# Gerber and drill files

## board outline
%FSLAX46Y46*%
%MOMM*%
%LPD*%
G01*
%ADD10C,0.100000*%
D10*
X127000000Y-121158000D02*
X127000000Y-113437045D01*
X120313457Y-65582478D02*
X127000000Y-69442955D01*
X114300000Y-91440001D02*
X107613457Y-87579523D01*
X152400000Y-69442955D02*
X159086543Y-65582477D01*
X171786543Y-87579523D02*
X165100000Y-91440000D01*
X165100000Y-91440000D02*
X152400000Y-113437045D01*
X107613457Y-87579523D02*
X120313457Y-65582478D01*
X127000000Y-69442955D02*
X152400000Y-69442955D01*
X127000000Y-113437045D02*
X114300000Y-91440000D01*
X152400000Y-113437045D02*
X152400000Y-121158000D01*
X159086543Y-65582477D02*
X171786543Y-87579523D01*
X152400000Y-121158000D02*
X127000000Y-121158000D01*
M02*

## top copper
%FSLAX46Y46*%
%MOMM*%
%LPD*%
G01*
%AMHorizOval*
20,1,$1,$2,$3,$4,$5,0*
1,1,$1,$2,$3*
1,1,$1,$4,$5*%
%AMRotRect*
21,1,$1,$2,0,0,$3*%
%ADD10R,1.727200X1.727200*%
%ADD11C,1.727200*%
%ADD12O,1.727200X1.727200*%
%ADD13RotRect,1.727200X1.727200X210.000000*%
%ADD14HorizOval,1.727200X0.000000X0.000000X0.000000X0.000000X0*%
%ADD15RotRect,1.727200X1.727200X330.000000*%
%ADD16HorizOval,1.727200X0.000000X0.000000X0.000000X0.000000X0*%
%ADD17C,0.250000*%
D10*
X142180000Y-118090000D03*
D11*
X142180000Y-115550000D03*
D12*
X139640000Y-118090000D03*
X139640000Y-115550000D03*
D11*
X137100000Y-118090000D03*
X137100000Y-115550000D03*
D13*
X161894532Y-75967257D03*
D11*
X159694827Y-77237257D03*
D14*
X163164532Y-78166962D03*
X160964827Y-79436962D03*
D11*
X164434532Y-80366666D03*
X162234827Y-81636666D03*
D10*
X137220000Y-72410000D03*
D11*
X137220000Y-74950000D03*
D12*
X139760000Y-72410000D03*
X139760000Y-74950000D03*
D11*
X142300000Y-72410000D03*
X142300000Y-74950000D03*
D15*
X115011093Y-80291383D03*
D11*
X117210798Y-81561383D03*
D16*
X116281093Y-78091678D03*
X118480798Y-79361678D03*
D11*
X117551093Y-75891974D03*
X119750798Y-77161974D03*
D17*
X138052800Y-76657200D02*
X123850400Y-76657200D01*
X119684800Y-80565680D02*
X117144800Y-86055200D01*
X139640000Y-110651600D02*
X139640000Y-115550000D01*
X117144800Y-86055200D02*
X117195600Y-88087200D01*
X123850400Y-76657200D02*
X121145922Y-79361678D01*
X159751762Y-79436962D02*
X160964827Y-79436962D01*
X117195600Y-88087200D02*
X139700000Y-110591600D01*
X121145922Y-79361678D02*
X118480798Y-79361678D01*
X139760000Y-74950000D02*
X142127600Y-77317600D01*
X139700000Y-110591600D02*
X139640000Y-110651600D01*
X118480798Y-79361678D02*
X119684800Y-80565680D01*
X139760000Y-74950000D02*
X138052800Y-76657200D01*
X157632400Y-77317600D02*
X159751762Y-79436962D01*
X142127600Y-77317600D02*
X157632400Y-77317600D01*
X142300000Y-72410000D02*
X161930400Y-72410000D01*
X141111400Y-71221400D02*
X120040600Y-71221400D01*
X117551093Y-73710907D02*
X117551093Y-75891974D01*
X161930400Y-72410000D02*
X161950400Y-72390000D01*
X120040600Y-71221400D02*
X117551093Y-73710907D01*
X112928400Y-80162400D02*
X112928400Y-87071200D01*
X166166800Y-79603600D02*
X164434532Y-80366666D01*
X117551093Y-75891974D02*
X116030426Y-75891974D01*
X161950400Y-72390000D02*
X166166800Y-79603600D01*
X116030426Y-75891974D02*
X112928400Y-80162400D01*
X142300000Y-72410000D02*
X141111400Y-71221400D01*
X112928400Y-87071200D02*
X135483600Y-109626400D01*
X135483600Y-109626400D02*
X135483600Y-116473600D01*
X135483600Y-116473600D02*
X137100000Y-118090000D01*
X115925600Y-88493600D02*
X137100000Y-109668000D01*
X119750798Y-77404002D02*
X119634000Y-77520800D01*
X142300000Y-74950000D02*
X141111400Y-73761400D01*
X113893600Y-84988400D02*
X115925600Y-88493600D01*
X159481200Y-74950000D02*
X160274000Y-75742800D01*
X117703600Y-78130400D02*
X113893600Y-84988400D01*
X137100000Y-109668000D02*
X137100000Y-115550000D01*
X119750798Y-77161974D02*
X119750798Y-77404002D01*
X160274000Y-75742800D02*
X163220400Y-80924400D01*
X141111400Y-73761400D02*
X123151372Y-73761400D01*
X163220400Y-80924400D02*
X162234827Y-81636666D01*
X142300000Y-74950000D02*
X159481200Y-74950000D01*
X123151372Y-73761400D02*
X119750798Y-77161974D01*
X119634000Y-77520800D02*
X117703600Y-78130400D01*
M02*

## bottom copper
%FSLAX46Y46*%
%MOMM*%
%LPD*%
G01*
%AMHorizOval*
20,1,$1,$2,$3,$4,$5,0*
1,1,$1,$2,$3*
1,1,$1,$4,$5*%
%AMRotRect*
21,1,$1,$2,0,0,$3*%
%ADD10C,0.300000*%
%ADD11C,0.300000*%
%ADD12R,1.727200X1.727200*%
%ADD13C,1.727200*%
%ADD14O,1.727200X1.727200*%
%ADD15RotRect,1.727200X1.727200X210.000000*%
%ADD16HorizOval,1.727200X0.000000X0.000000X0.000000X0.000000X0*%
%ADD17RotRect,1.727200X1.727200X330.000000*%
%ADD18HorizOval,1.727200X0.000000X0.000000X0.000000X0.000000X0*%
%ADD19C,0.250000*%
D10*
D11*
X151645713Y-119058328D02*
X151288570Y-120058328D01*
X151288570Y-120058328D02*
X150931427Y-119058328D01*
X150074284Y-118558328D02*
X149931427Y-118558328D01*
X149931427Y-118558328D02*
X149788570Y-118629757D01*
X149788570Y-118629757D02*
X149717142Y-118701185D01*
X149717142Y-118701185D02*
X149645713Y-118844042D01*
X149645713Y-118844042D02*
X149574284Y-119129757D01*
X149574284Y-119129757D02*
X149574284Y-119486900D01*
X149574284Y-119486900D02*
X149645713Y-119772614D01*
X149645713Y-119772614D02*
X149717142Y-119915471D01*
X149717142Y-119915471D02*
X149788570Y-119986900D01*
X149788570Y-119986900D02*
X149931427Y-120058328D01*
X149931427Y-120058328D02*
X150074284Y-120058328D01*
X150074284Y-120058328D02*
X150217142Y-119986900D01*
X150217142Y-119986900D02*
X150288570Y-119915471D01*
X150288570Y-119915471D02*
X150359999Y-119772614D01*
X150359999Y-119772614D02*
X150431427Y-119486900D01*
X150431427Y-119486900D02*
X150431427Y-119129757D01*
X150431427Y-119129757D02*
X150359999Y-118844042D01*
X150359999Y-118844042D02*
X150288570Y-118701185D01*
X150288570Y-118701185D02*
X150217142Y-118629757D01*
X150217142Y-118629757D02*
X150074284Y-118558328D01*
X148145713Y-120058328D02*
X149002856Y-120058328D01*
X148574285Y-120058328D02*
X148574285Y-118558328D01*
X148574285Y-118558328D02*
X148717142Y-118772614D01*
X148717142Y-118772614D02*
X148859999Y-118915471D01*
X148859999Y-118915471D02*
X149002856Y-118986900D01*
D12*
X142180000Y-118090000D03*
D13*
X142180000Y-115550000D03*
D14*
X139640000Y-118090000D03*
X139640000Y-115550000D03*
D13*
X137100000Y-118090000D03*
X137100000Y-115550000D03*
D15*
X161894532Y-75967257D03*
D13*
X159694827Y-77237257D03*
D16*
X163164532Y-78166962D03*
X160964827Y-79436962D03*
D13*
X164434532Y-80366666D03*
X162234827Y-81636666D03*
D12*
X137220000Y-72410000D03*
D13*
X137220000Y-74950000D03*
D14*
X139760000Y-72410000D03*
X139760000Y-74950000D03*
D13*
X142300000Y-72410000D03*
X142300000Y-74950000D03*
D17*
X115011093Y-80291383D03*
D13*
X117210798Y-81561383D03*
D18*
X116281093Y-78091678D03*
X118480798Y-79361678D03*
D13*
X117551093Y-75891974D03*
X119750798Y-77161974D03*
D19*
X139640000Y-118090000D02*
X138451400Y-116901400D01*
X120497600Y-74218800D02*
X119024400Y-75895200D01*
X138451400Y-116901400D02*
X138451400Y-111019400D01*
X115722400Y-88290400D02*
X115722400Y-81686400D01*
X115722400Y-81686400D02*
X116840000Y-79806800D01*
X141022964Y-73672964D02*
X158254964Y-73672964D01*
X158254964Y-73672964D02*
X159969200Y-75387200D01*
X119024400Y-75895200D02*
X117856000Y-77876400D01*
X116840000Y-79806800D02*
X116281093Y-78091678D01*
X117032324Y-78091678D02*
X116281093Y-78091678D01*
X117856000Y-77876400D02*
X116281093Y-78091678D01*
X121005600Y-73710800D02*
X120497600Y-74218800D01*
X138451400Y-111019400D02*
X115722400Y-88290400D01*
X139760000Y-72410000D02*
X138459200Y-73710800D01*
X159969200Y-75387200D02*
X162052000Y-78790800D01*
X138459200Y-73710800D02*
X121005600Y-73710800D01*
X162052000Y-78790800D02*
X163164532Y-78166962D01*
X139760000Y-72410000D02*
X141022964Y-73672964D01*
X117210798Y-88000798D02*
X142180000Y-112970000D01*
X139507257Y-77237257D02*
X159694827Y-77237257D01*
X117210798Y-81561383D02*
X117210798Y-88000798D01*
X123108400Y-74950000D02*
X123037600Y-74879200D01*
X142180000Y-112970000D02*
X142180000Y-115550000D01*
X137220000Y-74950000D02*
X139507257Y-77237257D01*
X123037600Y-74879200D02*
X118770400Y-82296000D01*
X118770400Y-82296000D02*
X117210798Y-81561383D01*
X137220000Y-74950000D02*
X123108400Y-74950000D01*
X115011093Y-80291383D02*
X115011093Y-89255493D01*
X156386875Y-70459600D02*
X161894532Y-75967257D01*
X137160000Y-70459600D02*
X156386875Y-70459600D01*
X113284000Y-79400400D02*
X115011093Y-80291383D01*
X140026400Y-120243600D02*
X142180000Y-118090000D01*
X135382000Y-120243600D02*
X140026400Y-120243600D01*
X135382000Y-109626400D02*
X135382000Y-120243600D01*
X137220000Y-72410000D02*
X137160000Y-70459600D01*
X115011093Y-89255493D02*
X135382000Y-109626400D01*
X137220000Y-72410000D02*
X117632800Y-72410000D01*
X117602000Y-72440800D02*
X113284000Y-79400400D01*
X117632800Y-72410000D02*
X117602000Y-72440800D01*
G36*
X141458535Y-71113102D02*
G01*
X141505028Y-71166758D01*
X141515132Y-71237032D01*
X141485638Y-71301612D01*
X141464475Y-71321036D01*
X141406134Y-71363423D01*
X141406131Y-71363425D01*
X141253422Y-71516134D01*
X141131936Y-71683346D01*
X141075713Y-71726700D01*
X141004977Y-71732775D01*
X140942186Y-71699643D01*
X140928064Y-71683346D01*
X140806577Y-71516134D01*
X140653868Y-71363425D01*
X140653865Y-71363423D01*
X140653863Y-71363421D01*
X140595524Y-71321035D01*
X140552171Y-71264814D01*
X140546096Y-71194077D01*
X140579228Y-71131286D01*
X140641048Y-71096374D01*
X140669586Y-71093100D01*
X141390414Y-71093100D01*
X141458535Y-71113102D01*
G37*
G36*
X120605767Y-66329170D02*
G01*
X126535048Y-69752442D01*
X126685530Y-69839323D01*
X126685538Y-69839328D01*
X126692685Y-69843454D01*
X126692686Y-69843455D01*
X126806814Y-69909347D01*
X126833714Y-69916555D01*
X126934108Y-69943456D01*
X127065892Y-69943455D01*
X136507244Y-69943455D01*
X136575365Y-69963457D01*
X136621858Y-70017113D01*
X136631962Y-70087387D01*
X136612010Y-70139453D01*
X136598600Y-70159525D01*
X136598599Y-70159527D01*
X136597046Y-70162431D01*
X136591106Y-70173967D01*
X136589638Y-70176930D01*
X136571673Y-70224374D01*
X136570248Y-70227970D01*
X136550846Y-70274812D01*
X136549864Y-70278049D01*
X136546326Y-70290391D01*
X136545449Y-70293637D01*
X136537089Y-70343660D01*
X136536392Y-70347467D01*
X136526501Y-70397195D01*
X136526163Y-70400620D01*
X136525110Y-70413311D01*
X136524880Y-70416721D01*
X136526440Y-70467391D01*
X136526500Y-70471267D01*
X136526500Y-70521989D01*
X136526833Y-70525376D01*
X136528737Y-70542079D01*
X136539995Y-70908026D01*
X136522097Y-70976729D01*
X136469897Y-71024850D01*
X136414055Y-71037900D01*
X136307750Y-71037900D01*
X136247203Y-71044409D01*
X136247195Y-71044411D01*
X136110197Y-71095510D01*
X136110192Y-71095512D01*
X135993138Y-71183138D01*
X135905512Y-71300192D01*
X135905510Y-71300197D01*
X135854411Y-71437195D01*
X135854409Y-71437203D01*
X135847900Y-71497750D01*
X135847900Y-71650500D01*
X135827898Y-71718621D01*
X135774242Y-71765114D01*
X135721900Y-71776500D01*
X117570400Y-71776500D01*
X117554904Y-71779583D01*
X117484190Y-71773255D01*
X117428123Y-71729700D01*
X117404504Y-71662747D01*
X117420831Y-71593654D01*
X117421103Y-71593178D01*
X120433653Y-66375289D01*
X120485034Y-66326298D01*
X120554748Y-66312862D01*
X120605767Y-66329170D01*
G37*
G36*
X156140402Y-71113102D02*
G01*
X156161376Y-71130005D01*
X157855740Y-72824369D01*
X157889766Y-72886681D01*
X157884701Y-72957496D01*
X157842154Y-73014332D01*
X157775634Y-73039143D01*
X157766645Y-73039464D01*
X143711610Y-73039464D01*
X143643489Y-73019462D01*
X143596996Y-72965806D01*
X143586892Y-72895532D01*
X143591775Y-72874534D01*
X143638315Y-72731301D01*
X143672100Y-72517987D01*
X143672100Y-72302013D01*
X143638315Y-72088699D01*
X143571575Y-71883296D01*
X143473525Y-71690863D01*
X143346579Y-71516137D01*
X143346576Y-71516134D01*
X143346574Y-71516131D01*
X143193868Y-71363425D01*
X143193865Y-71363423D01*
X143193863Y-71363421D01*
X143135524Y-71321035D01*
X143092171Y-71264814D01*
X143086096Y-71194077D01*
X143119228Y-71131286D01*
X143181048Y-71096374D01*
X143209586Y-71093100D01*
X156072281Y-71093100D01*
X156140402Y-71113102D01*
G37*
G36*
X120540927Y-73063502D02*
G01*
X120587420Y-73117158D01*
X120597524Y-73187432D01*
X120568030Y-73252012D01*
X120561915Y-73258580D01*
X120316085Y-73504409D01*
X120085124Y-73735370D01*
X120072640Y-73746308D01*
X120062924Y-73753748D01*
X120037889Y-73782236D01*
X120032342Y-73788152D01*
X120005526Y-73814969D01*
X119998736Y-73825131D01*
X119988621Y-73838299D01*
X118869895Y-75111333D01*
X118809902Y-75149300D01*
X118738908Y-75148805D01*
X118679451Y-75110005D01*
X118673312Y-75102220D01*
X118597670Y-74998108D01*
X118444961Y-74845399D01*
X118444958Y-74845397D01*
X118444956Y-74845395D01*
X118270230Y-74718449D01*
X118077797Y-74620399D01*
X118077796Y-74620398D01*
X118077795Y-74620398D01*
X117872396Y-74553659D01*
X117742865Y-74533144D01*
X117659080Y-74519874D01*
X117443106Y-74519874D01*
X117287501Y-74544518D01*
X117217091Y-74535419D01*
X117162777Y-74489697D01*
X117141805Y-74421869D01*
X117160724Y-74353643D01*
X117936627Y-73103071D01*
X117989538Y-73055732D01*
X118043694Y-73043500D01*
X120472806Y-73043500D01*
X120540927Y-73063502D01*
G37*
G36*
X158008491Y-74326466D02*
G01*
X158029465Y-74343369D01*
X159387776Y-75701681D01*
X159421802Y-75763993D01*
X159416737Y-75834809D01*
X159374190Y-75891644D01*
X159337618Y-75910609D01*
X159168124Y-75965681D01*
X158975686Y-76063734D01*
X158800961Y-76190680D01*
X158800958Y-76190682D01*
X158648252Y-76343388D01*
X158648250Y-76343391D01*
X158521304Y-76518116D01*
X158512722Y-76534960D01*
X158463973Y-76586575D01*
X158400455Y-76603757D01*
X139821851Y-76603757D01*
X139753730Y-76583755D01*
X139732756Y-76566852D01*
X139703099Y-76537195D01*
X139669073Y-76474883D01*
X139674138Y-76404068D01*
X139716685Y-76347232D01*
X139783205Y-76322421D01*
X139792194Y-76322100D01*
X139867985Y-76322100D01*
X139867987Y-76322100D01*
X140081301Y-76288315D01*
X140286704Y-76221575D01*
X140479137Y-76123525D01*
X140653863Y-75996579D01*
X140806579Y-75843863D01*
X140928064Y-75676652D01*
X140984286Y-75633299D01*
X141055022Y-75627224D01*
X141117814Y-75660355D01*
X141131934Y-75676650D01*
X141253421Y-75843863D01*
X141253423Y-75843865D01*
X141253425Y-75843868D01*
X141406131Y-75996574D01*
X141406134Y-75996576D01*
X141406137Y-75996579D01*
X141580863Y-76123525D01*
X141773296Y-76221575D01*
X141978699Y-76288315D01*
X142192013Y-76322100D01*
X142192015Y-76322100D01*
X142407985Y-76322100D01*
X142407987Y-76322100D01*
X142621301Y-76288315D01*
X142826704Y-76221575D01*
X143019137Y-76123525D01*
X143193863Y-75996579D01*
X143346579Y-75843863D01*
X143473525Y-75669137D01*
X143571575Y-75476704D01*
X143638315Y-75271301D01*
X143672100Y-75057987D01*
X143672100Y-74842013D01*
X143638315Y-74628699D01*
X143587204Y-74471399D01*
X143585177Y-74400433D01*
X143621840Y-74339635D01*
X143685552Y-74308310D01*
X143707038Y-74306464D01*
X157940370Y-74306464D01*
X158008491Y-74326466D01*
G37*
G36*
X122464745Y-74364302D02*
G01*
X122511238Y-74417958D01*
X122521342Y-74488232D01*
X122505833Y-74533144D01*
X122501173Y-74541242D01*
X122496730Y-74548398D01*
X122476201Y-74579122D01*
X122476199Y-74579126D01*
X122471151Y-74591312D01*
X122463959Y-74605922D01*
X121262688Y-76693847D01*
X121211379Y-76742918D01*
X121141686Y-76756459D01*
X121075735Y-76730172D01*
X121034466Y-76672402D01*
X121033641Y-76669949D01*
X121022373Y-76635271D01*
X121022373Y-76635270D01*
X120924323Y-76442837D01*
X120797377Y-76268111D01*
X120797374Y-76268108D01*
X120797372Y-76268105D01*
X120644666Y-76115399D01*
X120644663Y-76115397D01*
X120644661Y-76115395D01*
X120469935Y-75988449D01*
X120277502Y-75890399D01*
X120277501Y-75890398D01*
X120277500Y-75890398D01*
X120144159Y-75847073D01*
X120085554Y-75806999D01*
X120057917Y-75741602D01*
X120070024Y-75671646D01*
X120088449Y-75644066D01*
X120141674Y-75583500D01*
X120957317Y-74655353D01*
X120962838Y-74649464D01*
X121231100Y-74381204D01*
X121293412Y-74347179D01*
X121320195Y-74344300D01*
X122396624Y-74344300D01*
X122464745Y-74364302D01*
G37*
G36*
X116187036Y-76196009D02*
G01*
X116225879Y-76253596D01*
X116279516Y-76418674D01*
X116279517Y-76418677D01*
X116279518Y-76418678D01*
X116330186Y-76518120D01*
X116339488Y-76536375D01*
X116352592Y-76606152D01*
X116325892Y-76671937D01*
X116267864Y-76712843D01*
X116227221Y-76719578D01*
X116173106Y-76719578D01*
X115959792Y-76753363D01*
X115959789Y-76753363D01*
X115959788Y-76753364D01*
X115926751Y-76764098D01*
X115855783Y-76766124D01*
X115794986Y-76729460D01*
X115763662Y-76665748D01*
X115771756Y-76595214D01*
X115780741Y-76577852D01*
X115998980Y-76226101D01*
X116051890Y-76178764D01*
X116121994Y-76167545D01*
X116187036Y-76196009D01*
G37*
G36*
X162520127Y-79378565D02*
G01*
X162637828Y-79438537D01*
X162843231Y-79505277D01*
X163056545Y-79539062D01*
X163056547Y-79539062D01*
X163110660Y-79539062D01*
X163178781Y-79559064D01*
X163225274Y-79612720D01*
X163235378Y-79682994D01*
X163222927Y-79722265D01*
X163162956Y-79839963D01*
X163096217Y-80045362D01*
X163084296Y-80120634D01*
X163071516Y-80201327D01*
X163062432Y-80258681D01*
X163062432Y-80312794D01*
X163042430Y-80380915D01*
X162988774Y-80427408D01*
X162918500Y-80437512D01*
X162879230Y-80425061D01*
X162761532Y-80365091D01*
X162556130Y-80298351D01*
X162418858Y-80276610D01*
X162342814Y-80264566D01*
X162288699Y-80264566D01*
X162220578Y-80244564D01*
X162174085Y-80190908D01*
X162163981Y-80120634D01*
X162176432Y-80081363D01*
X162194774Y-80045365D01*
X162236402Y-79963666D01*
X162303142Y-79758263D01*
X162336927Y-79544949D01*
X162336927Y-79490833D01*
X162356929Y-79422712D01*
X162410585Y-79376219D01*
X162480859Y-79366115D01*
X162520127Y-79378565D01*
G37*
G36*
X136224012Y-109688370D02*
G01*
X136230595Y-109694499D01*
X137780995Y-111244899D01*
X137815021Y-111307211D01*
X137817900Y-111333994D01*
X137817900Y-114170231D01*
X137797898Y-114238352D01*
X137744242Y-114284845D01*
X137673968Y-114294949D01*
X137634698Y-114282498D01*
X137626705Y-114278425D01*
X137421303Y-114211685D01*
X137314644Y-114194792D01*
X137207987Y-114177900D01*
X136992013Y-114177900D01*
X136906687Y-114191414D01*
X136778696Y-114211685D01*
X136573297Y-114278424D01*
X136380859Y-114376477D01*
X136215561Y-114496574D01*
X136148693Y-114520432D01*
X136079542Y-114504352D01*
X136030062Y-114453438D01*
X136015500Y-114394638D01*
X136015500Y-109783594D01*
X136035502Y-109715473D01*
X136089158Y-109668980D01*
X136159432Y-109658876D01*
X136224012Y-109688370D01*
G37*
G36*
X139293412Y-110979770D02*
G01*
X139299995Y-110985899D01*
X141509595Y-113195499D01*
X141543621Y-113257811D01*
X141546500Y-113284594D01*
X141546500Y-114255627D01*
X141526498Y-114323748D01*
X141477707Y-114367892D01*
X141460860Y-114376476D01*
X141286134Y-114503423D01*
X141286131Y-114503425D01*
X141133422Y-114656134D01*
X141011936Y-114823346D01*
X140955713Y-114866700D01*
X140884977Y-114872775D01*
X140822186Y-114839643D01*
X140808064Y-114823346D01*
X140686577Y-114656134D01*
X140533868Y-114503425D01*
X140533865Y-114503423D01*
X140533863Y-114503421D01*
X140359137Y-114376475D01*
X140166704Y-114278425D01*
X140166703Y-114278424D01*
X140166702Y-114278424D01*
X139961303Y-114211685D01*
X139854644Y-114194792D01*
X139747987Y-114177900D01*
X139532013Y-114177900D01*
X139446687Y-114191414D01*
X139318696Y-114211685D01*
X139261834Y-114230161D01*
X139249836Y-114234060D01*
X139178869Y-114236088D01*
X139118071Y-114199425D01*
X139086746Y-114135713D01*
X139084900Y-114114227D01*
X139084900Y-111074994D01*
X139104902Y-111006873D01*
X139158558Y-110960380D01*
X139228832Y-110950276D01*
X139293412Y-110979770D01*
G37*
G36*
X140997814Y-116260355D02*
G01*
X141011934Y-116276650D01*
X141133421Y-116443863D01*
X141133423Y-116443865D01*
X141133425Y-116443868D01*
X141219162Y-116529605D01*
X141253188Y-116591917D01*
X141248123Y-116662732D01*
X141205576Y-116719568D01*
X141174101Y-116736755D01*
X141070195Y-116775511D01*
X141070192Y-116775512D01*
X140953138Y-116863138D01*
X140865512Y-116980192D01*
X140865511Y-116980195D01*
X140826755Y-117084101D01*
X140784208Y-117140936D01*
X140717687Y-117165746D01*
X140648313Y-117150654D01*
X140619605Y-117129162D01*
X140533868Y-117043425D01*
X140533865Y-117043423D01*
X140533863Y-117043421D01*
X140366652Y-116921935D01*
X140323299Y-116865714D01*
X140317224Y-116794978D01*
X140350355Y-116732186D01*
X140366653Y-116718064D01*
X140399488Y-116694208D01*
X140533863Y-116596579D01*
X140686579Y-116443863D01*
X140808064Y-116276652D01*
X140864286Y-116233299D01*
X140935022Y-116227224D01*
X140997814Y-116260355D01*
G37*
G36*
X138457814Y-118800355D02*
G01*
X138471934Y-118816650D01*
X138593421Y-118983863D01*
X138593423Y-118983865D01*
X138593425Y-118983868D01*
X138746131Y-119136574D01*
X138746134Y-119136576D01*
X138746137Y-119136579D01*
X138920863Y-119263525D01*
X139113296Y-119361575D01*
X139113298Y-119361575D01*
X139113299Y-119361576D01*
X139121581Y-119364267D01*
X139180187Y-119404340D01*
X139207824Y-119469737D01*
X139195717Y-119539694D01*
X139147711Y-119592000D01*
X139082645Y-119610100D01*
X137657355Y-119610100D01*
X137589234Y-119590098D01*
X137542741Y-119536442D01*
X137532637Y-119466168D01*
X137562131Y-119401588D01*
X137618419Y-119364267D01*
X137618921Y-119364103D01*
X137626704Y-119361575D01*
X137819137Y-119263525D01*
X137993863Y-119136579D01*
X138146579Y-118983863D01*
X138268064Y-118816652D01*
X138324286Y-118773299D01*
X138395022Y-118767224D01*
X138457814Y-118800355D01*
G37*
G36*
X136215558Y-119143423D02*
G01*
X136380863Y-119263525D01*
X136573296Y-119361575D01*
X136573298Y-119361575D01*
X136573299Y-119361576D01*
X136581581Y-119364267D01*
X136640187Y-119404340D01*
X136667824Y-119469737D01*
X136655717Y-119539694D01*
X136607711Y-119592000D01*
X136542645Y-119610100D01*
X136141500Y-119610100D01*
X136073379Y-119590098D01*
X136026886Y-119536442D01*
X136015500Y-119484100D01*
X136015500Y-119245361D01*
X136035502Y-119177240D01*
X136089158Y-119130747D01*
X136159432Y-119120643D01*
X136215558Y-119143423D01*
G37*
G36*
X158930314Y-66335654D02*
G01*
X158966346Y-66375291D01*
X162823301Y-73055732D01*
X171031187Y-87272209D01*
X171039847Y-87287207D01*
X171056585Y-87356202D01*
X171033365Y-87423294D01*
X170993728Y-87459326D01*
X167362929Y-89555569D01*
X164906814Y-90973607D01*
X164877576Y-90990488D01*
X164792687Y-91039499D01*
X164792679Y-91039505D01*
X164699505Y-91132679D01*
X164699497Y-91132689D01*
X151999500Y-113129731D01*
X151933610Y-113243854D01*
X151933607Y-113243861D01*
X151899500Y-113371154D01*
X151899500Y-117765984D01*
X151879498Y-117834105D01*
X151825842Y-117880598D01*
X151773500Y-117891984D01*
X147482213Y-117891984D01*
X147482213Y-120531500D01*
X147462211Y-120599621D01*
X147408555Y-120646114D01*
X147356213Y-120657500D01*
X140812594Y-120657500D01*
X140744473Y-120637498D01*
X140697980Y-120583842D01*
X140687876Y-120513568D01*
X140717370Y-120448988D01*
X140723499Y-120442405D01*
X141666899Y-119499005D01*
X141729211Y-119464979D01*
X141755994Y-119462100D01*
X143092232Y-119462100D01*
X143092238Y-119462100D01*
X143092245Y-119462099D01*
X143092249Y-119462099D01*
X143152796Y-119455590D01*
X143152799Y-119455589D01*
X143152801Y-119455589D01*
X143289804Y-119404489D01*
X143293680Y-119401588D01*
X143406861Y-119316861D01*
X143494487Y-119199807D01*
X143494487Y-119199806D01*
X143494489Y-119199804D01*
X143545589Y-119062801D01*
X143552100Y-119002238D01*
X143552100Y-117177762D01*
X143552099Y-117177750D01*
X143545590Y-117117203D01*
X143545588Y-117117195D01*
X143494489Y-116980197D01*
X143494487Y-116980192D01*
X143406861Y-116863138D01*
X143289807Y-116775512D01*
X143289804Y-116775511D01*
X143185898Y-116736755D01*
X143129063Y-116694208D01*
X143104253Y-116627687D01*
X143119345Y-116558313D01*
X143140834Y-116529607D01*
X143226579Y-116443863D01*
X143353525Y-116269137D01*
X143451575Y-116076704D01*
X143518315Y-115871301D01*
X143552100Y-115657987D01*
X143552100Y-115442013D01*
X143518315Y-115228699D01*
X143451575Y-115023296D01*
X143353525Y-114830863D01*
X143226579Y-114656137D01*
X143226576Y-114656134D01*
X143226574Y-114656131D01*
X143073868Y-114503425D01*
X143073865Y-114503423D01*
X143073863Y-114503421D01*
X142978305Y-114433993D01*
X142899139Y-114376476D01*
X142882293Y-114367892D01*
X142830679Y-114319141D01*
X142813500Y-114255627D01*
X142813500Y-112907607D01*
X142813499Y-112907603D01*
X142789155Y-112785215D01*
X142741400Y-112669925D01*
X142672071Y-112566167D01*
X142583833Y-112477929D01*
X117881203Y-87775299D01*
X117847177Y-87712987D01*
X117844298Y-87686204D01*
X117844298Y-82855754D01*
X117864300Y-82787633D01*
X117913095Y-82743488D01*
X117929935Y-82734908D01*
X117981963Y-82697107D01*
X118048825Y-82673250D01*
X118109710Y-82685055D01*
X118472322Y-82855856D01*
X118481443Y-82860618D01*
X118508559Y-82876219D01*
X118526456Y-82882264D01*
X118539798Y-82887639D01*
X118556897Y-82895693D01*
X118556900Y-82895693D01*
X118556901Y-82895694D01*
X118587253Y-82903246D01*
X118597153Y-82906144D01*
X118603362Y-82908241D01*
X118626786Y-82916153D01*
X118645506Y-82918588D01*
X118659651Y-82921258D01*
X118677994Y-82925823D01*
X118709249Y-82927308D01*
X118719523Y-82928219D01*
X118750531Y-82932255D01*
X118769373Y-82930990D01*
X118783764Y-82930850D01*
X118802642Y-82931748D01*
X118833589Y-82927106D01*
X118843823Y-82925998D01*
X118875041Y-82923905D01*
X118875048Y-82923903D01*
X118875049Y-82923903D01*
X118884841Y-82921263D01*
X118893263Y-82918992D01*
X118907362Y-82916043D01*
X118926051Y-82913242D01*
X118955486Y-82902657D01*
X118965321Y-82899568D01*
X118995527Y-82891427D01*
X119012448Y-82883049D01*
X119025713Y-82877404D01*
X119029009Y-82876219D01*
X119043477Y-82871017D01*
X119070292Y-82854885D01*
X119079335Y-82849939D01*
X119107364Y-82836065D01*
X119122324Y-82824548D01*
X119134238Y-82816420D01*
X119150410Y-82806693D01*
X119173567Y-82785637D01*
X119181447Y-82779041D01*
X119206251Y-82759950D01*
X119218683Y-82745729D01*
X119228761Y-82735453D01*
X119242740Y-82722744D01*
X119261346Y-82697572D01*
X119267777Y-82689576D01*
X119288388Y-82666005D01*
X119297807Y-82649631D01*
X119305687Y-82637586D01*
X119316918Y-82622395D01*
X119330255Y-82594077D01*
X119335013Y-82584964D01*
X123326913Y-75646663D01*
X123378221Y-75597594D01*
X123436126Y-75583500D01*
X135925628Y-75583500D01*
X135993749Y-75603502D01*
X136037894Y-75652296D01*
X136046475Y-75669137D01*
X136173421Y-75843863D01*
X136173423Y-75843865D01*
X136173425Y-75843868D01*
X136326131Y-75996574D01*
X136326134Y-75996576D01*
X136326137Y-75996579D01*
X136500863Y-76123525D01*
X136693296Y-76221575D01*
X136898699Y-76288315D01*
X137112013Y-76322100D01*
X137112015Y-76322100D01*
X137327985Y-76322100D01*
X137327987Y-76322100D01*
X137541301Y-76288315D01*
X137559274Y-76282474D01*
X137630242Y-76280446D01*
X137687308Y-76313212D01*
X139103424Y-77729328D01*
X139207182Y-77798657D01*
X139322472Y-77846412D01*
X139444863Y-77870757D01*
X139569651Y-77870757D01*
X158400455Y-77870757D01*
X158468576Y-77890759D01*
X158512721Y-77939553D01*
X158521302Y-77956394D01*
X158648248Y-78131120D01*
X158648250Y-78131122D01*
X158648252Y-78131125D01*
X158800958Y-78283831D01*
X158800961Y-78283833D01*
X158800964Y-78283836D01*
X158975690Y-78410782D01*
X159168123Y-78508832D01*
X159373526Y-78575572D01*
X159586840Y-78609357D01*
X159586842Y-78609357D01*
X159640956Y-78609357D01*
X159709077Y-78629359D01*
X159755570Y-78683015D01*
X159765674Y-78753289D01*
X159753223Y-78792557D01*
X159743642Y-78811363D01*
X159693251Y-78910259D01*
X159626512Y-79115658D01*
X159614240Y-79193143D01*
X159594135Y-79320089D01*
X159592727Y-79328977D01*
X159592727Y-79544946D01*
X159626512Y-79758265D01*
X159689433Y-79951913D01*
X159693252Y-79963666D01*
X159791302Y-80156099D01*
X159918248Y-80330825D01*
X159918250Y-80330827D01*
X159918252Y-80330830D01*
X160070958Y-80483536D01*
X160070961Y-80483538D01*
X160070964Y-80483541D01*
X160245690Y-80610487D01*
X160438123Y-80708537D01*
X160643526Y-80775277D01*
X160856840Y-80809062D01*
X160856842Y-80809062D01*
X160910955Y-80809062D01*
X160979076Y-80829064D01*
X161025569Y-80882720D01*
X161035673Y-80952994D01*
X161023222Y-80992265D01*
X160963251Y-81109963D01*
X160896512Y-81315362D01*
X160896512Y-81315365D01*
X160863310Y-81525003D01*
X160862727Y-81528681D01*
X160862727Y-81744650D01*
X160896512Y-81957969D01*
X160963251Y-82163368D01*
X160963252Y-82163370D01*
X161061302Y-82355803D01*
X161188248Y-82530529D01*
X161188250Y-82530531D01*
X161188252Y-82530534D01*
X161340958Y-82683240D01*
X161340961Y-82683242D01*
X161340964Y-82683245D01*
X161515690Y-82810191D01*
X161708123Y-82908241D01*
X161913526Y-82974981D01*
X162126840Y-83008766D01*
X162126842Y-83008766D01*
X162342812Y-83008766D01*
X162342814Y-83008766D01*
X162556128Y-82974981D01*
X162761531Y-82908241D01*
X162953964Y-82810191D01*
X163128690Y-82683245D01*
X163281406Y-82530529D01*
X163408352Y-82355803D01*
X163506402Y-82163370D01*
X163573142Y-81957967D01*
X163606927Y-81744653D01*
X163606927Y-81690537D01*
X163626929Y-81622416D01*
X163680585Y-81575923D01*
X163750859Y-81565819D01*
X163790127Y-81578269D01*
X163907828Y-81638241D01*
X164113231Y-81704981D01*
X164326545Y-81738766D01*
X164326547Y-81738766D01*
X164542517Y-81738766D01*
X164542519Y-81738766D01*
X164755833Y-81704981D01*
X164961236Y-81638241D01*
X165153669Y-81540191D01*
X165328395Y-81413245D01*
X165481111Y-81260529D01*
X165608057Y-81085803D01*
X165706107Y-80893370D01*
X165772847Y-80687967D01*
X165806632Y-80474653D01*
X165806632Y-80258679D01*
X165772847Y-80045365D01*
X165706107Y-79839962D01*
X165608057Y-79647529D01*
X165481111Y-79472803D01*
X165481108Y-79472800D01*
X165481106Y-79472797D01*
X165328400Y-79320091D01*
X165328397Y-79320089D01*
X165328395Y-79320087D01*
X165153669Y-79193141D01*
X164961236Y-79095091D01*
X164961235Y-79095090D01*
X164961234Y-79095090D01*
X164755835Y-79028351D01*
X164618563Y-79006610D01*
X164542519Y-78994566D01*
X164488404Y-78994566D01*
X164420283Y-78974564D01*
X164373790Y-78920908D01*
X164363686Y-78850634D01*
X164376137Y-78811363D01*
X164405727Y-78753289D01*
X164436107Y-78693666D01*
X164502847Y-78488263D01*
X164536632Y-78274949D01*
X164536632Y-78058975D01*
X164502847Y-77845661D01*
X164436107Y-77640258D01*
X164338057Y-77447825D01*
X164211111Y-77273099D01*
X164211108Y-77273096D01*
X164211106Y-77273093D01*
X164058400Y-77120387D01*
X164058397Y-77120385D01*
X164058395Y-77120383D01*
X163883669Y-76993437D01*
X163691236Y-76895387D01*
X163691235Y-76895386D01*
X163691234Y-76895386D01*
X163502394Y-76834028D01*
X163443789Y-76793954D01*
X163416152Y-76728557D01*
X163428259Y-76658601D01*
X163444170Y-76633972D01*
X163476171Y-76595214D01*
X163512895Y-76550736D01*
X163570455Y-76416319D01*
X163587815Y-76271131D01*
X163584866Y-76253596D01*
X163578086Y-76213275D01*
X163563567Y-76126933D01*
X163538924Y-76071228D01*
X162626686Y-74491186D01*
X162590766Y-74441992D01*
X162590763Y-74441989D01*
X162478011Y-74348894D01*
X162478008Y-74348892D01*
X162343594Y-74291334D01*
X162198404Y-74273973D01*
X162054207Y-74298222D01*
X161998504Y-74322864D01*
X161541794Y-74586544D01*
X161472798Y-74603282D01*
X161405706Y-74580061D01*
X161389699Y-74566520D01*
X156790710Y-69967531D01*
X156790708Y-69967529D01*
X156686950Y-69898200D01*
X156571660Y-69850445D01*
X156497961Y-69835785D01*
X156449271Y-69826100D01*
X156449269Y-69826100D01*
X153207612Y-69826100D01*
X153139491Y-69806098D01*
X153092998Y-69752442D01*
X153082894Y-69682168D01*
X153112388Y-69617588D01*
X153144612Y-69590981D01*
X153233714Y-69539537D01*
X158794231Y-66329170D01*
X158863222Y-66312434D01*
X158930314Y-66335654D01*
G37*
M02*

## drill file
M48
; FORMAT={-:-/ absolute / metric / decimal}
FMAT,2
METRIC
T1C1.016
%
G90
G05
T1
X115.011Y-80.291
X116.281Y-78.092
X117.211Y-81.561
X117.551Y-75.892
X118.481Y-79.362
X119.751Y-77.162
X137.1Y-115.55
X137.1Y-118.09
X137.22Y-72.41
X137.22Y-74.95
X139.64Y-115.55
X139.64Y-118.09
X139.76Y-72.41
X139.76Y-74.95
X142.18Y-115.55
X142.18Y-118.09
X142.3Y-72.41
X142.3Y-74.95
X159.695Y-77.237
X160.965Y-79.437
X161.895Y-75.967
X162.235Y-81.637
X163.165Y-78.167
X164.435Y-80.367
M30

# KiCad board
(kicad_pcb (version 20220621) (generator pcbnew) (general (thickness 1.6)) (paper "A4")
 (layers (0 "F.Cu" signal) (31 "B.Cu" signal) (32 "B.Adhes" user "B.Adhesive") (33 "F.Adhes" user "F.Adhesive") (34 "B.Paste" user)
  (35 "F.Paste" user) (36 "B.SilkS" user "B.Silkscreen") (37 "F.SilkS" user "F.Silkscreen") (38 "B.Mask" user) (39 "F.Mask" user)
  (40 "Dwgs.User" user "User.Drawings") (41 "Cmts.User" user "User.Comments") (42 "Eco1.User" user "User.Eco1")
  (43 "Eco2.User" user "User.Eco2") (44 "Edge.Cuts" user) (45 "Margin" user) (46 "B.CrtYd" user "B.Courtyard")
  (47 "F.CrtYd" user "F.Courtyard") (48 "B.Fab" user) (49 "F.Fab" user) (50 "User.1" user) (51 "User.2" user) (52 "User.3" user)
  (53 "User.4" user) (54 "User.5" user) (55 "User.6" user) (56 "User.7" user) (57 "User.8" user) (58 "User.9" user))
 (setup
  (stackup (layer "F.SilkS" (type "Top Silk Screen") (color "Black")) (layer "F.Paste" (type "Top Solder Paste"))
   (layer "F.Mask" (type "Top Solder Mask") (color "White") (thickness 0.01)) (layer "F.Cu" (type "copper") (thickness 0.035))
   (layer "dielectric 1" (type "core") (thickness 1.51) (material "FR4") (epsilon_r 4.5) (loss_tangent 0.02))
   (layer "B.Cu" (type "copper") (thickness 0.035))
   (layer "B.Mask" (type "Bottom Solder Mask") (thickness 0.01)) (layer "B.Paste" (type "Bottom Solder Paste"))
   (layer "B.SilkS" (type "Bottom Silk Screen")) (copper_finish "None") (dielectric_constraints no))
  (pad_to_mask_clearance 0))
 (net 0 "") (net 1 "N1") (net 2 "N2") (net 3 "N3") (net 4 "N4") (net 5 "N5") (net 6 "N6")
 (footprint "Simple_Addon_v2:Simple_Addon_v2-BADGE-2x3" (layer "F.Cu") (at 139.7 116.84 180)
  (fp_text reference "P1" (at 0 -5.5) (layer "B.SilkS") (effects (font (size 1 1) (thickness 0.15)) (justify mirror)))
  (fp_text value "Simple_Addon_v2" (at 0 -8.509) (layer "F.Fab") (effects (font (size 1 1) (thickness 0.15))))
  (pad "1" thru_hole rect locked (at -2.48 -1.25 90) (size 1.7272 1.7272) (drill 1.016) (layers *.Cu *.Mask) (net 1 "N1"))
  (pad "2" thru_hole circle locked (at -2.48 1.29 90) (size 1.7272 1.7272) (drill 1.016) (layers *.Cu *.Mask) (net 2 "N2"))
  (pad "3" thru_hole oval locked (at 0.06 -1.25 90) (size 1.7272 1.7272) (drill 1.016) (layers *.Cu *.Mask) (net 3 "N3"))
  (pad "4" thru_hole oval locked (at 0.06 1.29 90) (size 1.7272 1.7272) (drill 1.016) (layers *.Cu *.Mask) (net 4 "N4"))
  (pad "5" thru_hole circle locked (at 2.6 -1.25 90) (size 1.7272 1.7272) (drill 1.016) (layers *.Cu *.Mask) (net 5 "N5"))
  (pad "6" thru_hole circle locked (at 2.6 1.29 90) (size 1.7272 1.7272) (drill 1.016) (layers *.Cu *.Mask) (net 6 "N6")))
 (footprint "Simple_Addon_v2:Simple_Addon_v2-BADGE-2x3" (layer "F.Cu") (at 162.052 78.74 -60)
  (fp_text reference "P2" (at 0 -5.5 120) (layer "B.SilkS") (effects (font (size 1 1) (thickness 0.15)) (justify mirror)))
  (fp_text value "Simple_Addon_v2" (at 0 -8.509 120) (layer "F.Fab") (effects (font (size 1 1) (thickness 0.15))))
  (pad "1" thru_hole rect locked (at -2.48 -1.25 210) (size 1.7272 1.7272) (drill 1.016) (layers *.Cu *.Mask) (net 1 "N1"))
  (pad "2" thru_hole circle locked (at -2.48 1.29 210) (size 1.7272 1.7272) (drill 1.016) (layers *.Cu *.Mask) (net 2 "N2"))
  (pad "3" thru_hole oval locked (at 0.06 -1.25 210) (size 1.7272 1.7272) (drill 1.016) (layers *.Cu *.Mask) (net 3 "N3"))
  (pad "4" thru_hole oval locked (at 0.06 1.29 210) (size 1.7272 1.7272) (drill 1.016) (layers *.Cu *.Mask) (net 4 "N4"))
  (pad "5" thru_hole circle locked (at 2.6 -1.25 210) (size 1.7272 1.7272) (drill 1.016) (layers *.Cu *.Mask) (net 5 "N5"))
  (pad "6" thru_hole circle locked (at 2.6 1.29 210) (size 1.7272 1.7272) (drill 1.016) (layers *.Cu *.Mask) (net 6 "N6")))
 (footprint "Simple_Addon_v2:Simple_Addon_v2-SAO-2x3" (layer "F.Cu") (at 139.7 73.66)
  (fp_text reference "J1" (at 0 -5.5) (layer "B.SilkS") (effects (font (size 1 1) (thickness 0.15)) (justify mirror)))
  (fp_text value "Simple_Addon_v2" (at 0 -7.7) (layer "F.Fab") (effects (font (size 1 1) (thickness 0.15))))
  (pad "1" thru_hole rect locked (at -2.48 -1.25 270) (size 1.7272 1.7272) (drill 1.016) (layers *.Cu *.Mask) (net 1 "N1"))
  (pad "2" thru_hole circle locked (at -2.48 1.29 270) (size 1.7272 1.7272) (drill 1.016) (layers *.Cu *.Mask) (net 2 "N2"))
  (pad "3" thru_hole oval locked (at 0.06 -1.25 270) (size 1.7272 1.7272) (drill 1.016) (layers *.Cu *.Mask) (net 3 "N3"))
  (pad "4" thru_hole oval locked (at 0.06 1.29 270) (size 1.7272 1.7272) (drill 1.016) (layers *.Cu *.Mask) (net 4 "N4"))
  (pad "5" thru_hole circle locked (at 2.6 -1.25 270) (size 1.7272 1.7272) (drill 1.016) (layers *.Cu *.Mask) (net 5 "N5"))
  (pad "6" thru_hole circle locked (at 2.6 1.29 270) (size 1.7272 1.7272) (drill 1.016) (layers *.Cu *.Mask) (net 6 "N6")))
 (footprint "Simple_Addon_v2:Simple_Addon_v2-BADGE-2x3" (layer "F.Cu") (at 117.333625 78.76864 60)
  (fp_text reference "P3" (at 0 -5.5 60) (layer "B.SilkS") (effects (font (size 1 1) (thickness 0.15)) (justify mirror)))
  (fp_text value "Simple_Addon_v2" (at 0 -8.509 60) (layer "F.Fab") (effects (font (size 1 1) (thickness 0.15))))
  (pad "1" thru_hole rect locked (at -2.48 -1.25 330) (size 1.7272 1.7272) (drill 1.016) (layers *.Cu *.Mask) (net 1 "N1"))
  (pad "2" thru_hole circle locked (at -2.48 1.29 330) (size 1.7272 1.7272) (drill 1.016) (layers *.Cu *.Mask) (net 2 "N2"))
  (pad "3" thru_hole oval locked (at 0.06 -1.25 330) (size 1.7272 1.7272) (drill 1.016) (layers *.Cu *.Mask) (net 3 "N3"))
  (pad "4" thru_hole oval locked (at 0.06 1.29 330) (size 1.7272 1.7272) (drill 1.016) (layers *.Cu *.Mask) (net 4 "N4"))
  (pad "5" thru_hole circle locked (at 2.6 -1.25 330) (size 1.7272 1.7272) (drill 1.016) (layers *.Cu *.Mask) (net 5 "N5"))
  (pad "6" thru_hole circle locked (at 2.6 1.29 330) (size 1.7272 1.7272) (drill 1.016) (layers *.Cu *.Mask) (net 6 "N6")))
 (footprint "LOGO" (layer "F.Cu") (at 140.97 91.44)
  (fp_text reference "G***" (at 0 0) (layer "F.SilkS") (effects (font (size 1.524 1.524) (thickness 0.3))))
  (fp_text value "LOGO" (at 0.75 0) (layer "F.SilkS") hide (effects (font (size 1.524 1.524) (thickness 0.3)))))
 (gr_line (start 127 121.158) (end 127 113.437045) (stroke (width 0.1) (type solid)) (layer "Edge.Cuts"))
 (gr_line (start 120.313457 65.582478) (end 127 69.442955) (stroke (width 0.1) (type solid)) (layer "Edge.Cuts"))
 (gr_line (start 114.3 91.440001) (end 107.613457 87.579523) (stroke (width 0.1) (type solid)) (layer "Edge.Cuts"))
 (gr_line (start 152.4 69.442955) (end 159.086543 65.582477) (stroke (width 0.1) (type solid)) (layer "Edge.Cuts"))
 (gr_line (start 171.786543 87.579523) (end 165.1 91.44) (stroke (width 0.1) (type solid)) (layer "Edge.Cuts"))
 (gr_line (start 165.1 91.44) (end 152.4 113.437045) (stroke (width 0.1) (type solid)) (layer "Edge.Cuts"))
 (gr_line (start 107.613457 87.579523) (end 120.313457 65.582478) (stroke (width 0.1) (type solid)) (layer "Edge.Cuts"))
 (gr_line (start 127 69.442955) (end 152.4 69.442955) (stroke (width 0.1) (type solid)) (layer "Edge.Cuts"))
 (gr_line (start 127 113.437045) (end 114.3 91.44) (stroke (width 0.1) (type solid)) (layer "Edge.Cuts"))
 (gr_line (start 152.4 113.437045) (end 152.4 121.158) (stroke (width 0.1) (type solid)) (layer "Edge.Cuts"))
 (gr_line (start 159.086543 65.582477) (end 171.786543 87.579523) (stroke (width 0.1) (type solid)) (layer "Edge.Cuts"))
 (gr_line (start 152.4 121.158) (end 127 121.158) (stroke (width 0.1) (type solid)) (layer "Edge.Cuts"))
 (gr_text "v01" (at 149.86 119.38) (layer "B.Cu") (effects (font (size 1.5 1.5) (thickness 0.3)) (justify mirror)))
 (segment (start 139.64 118.09) (end 138.4514 116.9014) (width 0.25) (layer "B.Cu") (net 3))
 (segment (start 120.4976 74.2188) (end 119.0244 75.8952) (width 0.25) (layer "B.Cu") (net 3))
 (segment (start 138.4514 116.9014) (end 138.4514 111.0194) (width 0.25) (layer "B.Cu") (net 3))
 (segment (start 115.7224 88.2904) (end 115.7224 81.6864) (width 0.25) (layer "B.Cu") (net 3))
 (segment (start 115.7224 81.6864) (end 116.84 79.8068) (width 0.25) (layer "B.Cu") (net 3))
 (segment (start 141.022964 73.672964) (end 158.254964 73.672964) (width 0.25) (layer "B.Cu") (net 3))
 (segment (start 158.254964 73.672964) (end 159.9692 75.3872) (width 0.25) (layer "B.Cu") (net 3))
 (segment (start 119.0244 75.8952) (end 117.856 77.8764) (width 0.25) (layer "B.Cu") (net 3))
 (segment (start 116.84 79.8068) (end 116.281093 78.091678) (width 0.25) (layer "B.Cu") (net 3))
 (segment (start 117.032324 78.091678) (end 116.281093 78.091678) (width 0.25) (layer "B.Cu") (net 3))
 (segment (start 117.856 77.8764) (end 116.281093 78.091678) (width 0.25) (layer "B.Cu") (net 3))
 (segment (start 121.0056 73.7108) (end 120.4976 74.2188) (width 0.25) (layer "B.Cu") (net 3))
 (segment (start 138.4514 111.0194) (end 115.7224 88.2904) (width 0.25) (layer "B.Cu") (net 3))
 (segment (start 139.76 72.41) (end 138.4592 73.7108) (width 0.25) (layer "B.Cu") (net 3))
 (segment (start 159.9692 75.3872) (end 162.052 78.7908) (width 0.25) (layer "B.Cu") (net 3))
 (segment (start 138.4592 73.7108) (end 121.0056 73.7108) (width 0.25) (layer "B.Cu") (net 3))
 (segment (start 162.052 78.7908) (end 163.164532 78.166962) (width 0.25) (layer "B.Cu") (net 3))
 (segment (start 139.76 72.41) (end 141.022964 73.672964) (width 0.25) (layer "B.Cu") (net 3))
 (segment (start 117.210798 88.000798) (end 142.18 112.97) (width 0.25) (layer "B.Cu") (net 2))
 (segment (start 139.507257 77.237257) (end 159.694827 77.237257) (width 0.25) (layer "B.Cu") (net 2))
 (segment (start 117.210798 81.561383) (end 117.210798 88.000798) (width 0.25) (layer "B.Cu") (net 2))
 (segment (start 123.1084 74.95) (end 123.0376 74.8792) (width 0.25) (layer "B.Cu") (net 2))
 (segment (start 142.18 112.97) (end 142.18 115.55) (width 0.25) (layer "B.Cu") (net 2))
 (segment (start 137.22 74.95) (end 139.507257 77.237257) (width 0.25) (layer "B.Cu") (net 2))
 (segment (start 123.0376 74.8792) (end 118.7704 82.296) (width 0.25) (layer "B.Cu") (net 2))
 (segment (start 118.7704 82.296) (end 117.210798 81.561383) (width 0.25) (layer "B.Cu") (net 2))
 (segment (start 137.22 74.95) (end 123.1084 74.95) (width 0.25) (layer "B.Cu") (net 2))
 (segment (start 138.0528 76.6572) (end 123.8504 76.6572) (width 0.25) (layer "F.Cu") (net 4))
 (segment (start 119.6848 80.56568) (end 117.1448 86.0552) (width 0.25) (layer "F.Cu") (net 4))
 (segment (start 139.64 110.6516) (end 139.64 115.55) (width 0.25) (layer "F.Cu") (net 4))
 (segment (start 117.1448 86.0552) (end 117.1956 88.0872) (width 0.25) (layer "F.Cu") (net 4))
 (segment (start 123.8504 76.6572) (end 121.145922 79.361678) (width 0.25) (layer "F.Cu") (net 4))
 (segment (start 159.751762 79.436962) (end 160.964827 79.436962) (width 0.25) (layer "F.Cu") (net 4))
 (segment (start 117.1956 88.0872) (end 139.7 110.5916) (width 0.25) (layer "F.Cu") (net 4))
 (segment (start 121.145922 79.361678) (end 118.480798 79.361678) (width 0.25) (layer "F.Cu") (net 4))
 (segment (start 139.76 74.95) (end 142.1276 77.3176) (width 0.25) (layer "F.Cu") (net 4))
 (segment (start 139.7 110.5916) (end 139.64 110.6516) (width 0.25) (layer "F.Cu") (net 4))
 (segment (start 118.480798 79.361678) (end 119.6848 80.56568) (width 0.25) (layer "F.Cu") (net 4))
 (segment (start 139.76 74.95) (end 138.0528 76.6572) (width 0.25) (layer "F.Cu") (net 4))
 (segment (start 157.6324 77.3176) (end 159.751762 79.436962) (width 0.25) (layer "F.Cu") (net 4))
 (segment (start 142.1276 77.3176) (end 157.6324 77.3176) (width 0.25) (layer "F.Cu") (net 4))
 (segment (start 115.011093 80.291383) (end 115.011093 89.255493) (width 0.25) (layer "B.Cu") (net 1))
 (segment (start 156.386875 70.4596) (end 161.894532 75.967257) (width 0.25) (layer "B.Cu") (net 1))
 (segment (start 137.16 70.4596) (end 156.386875 70.4596) (width 0.25) (layer "B.Cu") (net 1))
 (segment (start 113.284 79.4004) (end 115.011093 80.291383) (width 0.25) (layer "B.Cu") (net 1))
 (segment (start 140.0264 120.2436) (end 142.18 118.09) (width 0.25) (layer "B.Cu") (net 1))
 (segment (start 135.382 120.2436) (end 140.0264 120.2436) (width 0.25) (layer "B.Cu") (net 1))
 (segment (start 135.382 109.6264) (end 135.382 120.2436) (width 0.25) (layer "B.Cu") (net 1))
 (segment (start 137.22 72.41) (end 137.16 70.4596) (width 0.25) (layer "B.Cu") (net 1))
 (segment (start 115.011093 89.255493) (end 135.382 109.6264) (width 0.25) (layer "B.Cu") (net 1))
 (segment (start 137.22 72.41) (end 117.6328 72.41) (width 0.25) (layer "B.Cu") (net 1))
 (segment (start 117.602 72.4408) (end 113.284 79.4004) (width 0.25) (layer "B.Cu") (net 1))
 (segment (start 117.6328 72.41) (end 117.602 72.4408) (width 0.25) (layer "B.Cu") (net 1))
 (segment (start 142.3 72.41) (end 161.9304 72.41) (width 0.25) (layer "F.Cu") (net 5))
 (segment (start 141.1114 71.2214) (end 120.0406 71.2214) (width 0.25) (layer "F.Cu") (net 5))
 (segment (start 117.551093 73.710907) (end 117.551093 75.891974) (width 0.25) (layer "F.Cu") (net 5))
 (segment (start 161.9304 72.41) (end 161.9504 72.39) (width 0.25) (layer "F.Cu") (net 5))
 (segment (start 120.0406 71.2214) (end 117.551093 73.710907) (width 0.25) (layer "F.Cu") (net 5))
 (segment (start 112.9284 80.1624) (end 112.9284 87.0712) (width 0.25) (layer "F.Cu") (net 5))
 (segment (start 166.1668 79.6036) (end 164.434532 80.366666) (width 0.25) (layer "F.Cu") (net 5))
 (segment (start 117.551093 75.891974) (end 116.030426 75.891974) (width 0.25) (layer "F.Cu") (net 5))
 (segment (start 161.9504 72.39) (end 166.1668 79.6036) (width 0.25) (layer "F.Cu") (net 5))
 (segment (start 116.030426 75.891974) (end 112.9284 80.1624) (width 0.25) (layer "F.Cu") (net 5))
 (segment (start 142.3 72.41) (end 141.1114 71.2214) (width 0.25) (layer "F.Cu") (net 5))
 (segment (start 112.9284 87.0712) (end 135.4836 109.6264) (width 0.25) (layer "F.Cu") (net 5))
 (segment (start 135.4836 109.6264) (end 135.4836 116.4736) (width 0.25) (layer "F.Cu") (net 5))
 (segment (start 135.4836 116.4736) (end 137.1 118.09) (width 0.25) (layer "F.Cu") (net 5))
 (segment (start 115.9256 88.4936) (end 137.1 109.668) (width 0.25) (layer "F.Cu") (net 6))
 (segment (start 119.750798 77.404002) (end 119.634 77.5208) (width 0.25) (layer "F.Cu") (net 6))
 (segment (start 142.3 74.95) (end 141.1114 73.7614) (width 0.25) (layer "F.Cu") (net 6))
 (segment (start 113.8936 84.9884) (end 115.9256 88.4936) (width 0.25) (layer "F.Cu") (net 6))
 (segment (start 159.4812 74.95) (end 160.274 75.7428) (width 0.25) (layer "F.Cu") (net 6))
 (segment (start 117.7036 78.1304) (end 113.8936 84.9884) (width 0.25) (layer "F.Cu") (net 6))
 (segment (start 137.1 109.668) (end 137.1 115.55) (width 0.25) (layer "F.Cu") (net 6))
 (segment (start 119.750798 77.161974) (end 119.750798 77.404002) (width 0.25) (layer "F.Cu") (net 6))
 (segment (start 160.274 75.7428) (end 163.2204 80.9244) (width 0.25) (layer "F.Cu") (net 6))
 (segment (start 141.1114 73.7614) (end 123.151372 73.7614) (width 0.25) (layer "F.Cu") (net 6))
 (segment (start 163.2204 80.9244) (end 162.234827 81.636666) (width 0.25) (layer "F.Cu") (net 6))
 (segment (start 142.3 74.95) (end 159.4812 74.95) (width 0.25) (layer "F.Cu") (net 6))
 (segment (start 123.151372 73.7614) (end 119.750798 77.161974) (width 0.25) (layer "F.Cu") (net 6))
 (segment (start 119.634 77.5208) (end 117.7036 78.1304) (width 0.25) (layer "F.Cu") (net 6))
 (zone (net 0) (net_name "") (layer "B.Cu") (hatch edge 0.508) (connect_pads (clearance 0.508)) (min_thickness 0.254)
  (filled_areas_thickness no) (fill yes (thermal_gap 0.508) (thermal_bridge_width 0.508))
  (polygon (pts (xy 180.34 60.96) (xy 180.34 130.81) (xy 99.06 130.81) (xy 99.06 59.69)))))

